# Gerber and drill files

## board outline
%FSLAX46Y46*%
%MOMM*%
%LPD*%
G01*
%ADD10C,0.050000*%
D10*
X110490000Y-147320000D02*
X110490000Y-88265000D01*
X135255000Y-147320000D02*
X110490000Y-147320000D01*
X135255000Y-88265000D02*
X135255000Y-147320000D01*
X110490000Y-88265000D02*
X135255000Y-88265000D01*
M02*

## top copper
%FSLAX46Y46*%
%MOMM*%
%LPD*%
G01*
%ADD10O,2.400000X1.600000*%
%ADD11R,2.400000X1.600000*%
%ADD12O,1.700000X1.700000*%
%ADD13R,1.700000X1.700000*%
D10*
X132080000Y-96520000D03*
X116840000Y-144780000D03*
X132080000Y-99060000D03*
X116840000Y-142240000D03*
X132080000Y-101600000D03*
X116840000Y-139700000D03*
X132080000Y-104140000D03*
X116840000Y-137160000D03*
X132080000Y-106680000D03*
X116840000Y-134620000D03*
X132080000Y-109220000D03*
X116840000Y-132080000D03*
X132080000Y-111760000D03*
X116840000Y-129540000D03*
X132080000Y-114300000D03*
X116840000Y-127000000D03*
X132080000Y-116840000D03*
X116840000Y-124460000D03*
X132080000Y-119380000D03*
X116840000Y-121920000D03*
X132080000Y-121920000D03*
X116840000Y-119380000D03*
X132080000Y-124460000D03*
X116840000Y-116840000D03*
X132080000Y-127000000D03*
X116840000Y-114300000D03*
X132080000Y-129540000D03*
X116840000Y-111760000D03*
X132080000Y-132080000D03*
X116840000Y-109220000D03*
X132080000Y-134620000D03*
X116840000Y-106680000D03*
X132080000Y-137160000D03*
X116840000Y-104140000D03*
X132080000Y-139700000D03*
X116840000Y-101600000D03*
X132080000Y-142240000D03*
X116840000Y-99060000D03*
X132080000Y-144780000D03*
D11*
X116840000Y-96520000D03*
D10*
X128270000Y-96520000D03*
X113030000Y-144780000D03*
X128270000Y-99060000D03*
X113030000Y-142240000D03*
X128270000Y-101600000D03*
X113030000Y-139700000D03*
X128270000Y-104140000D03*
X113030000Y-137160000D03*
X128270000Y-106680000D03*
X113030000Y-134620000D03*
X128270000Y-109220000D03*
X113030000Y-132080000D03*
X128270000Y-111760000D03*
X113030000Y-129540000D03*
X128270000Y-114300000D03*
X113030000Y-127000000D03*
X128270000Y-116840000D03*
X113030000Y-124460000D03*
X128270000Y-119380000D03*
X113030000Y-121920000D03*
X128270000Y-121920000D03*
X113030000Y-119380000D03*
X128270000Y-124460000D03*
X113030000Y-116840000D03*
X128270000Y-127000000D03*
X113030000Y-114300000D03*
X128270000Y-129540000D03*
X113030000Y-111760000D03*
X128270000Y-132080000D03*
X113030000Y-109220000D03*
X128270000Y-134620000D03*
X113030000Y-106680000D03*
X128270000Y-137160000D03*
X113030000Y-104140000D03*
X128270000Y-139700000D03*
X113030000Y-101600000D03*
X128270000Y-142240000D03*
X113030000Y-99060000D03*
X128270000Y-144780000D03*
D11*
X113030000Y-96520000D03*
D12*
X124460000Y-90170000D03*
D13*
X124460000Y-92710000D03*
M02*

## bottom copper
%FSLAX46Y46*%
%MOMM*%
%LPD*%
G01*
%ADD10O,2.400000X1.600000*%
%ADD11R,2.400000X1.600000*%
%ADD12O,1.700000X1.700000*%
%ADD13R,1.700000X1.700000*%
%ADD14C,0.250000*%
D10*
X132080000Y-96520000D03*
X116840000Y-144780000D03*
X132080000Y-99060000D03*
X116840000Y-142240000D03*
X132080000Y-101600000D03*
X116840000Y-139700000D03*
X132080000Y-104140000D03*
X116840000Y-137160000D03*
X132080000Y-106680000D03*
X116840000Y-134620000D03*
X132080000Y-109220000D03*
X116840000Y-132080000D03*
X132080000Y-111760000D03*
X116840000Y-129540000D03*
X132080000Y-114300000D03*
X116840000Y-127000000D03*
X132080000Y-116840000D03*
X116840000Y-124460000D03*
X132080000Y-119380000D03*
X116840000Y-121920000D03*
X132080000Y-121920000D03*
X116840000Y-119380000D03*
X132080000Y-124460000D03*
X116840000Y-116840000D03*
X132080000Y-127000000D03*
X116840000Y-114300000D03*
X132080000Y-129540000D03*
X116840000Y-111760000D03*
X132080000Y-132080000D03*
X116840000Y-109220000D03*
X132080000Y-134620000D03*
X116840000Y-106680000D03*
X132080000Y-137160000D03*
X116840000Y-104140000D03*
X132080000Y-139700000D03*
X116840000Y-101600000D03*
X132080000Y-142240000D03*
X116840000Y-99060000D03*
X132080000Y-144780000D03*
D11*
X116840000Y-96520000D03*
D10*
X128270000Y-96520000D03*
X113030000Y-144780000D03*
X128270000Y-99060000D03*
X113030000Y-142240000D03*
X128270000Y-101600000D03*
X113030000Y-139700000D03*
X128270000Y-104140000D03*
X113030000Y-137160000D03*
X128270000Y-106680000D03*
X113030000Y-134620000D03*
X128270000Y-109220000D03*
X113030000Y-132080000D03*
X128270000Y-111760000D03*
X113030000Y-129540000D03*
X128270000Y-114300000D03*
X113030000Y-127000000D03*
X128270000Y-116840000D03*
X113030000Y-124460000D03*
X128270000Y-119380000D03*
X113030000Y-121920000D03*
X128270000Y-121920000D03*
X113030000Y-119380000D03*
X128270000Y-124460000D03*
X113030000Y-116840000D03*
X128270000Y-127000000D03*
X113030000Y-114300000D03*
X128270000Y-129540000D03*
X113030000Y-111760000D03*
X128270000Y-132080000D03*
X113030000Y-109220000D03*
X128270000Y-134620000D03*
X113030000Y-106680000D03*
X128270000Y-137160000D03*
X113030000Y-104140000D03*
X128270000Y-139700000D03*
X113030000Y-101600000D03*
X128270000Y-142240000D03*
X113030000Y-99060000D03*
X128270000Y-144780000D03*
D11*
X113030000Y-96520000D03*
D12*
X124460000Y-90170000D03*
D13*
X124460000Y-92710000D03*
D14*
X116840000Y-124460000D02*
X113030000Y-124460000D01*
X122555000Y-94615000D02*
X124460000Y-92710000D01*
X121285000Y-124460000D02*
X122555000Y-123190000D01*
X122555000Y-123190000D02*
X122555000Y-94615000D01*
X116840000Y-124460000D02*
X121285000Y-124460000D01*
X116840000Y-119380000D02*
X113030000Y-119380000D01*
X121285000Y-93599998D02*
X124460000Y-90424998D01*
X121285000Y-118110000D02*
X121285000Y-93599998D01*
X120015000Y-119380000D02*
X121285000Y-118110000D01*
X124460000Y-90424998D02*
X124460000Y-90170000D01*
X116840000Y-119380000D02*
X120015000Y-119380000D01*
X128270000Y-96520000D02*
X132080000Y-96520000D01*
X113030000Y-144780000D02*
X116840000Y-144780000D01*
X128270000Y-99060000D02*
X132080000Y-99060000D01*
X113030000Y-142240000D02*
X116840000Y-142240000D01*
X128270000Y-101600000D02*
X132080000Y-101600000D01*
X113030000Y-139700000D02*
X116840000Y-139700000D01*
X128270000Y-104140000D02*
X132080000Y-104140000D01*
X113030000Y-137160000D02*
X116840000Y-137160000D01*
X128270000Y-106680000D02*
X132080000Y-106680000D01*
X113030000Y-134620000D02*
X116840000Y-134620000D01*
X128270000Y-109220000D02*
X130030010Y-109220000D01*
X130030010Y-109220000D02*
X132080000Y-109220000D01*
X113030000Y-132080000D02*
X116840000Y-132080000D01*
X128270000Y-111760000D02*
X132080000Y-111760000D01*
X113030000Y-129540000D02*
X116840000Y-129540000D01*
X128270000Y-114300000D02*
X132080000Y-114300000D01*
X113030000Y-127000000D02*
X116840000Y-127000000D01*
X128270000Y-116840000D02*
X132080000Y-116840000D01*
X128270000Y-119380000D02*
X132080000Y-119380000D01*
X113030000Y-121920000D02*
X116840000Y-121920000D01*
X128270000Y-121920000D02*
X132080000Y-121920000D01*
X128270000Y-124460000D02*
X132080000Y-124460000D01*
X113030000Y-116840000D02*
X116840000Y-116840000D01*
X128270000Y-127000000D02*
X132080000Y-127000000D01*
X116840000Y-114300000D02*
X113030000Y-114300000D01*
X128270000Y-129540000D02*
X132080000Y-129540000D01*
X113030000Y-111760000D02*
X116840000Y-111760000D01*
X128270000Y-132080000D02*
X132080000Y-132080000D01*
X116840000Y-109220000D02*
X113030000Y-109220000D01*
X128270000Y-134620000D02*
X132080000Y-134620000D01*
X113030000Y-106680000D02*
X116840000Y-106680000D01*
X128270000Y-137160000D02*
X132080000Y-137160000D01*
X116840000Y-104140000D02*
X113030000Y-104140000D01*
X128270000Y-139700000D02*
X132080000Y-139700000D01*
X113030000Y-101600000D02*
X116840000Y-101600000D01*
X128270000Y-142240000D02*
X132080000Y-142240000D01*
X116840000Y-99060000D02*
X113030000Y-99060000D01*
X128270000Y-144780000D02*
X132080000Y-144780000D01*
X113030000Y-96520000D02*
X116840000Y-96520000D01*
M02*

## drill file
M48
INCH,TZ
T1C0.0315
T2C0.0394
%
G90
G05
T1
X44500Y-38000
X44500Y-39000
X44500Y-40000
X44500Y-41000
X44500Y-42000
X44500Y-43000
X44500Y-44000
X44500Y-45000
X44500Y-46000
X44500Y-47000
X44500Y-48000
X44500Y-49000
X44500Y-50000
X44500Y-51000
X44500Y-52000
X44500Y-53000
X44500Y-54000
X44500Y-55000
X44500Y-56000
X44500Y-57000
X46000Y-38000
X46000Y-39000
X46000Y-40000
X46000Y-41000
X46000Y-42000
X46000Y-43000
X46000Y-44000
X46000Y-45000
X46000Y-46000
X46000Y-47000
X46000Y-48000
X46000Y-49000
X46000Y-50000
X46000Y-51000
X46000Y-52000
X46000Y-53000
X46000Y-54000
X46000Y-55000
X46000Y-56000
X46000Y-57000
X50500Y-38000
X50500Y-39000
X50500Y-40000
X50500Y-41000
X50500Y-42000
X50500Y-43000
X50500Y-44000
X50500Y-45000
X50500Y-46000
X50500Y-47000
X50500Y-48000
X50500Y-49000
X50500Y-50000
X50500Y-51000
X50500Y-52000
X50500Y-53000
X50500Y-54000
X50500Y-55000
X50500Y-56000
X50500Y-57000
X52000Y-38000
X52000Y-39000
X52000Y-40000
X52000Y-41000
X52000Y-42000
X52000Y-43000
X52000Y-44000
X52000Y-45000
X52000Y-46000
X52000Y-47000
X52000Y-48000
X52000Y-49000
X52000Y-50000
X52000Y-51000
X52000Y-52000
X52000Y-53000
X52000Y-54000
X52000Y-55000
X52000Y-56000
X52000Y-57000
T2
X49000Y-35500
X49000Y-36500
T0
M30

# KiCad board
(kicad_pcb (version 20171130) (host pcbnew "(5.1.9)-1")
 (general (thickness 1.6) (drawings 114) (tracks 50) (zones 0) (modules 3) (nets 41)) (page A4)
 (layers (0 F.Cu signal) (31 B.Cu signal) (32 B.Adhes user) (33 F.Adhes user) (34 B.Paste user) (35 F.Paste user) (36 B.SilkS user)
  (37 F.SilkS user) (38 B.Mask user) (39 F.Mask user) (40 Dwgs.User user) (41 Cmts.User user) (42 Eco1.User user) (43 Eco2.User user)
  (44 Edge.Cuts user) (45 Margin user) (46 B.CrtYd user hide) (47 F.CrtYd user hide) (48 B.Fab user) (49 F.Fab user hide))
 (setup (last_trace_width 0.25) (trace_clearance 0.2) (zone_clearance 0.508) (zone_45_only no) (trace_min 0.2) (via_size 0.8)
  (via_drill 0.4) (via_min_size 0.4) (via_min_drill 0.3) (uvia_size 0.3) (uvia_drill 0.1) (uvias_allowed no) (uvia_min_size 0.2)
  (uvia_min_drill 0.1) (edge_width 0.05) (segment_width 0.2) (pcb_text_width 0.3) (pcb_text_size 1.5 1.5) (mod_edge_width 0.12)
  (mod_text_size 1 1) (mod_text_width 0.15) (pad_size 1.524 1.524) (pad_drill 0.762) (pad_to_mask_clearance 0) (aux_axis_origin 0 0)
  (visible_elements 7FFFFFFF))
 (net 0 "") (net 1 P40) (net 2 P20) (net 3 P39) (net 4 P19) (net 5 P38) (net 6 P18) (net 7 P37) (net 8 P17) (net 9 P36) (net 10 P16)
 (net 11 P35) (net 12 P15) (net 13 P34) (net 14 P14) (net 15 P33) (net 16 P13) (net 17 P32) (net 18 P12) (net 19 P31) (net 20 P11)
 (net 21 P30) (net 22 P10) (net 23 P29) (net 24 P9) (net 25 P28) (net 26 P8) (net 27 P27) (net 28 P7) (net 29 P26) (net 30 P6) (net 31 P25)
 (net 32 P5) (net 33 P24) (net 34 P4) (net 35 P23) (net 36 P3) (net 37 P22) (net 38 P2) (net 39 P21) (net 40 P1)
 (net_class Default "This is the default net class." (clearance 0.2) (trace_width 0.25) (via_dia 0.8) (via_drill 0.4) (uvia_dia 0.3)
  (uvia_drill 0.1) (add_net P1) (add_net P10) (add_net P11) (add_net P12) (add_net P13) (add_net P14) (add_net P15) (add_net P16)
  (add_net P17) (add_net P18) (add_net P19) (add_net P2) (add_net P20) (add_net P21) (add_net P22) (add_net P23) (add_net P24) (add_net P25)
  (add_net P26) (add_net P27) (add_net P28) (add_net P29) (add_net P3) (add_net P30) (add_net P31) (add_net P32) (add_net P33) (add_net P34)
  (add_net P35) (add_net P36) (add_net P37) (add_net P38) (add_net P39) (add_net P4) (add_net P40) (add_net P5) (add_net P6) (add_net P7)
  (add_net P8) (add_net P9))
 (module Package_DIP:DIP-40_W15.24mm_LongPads (layer F.Cu) (at 116.84 96.52)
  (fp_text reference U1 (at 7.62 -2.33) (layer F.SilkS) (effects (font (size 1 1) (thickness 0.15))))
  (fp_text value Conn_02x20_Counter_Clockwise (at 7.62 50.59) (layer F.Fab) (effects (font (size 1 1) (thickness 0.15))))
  (pad 40 thru_hole oval (at 15.24 0) (size 2.4 1.6) (drill 0.8) (layers *.Cu *.Mask) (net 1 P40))
  (pad 20 thru_hole oval (at 0 48.26) (size 2.4 1.6) (drill 0.8) (layers *.Cu *.Mask) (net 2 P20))
  (pad 39 thru_hole oval (at 15.24 2.54) (size 2.4 1.6) (drill 0.8) (layers *.Cu *.Mask) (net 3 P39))
  (pad 19 thru_hole oval (at 0 45.72) (size 2.4 1.6) (drill 0.8) (layers *.Cu *.Mask) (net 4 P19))
  (pad 38 thru_hole oval (at 15.24 5.08) (size 2.4 1.6) (drill 0.8) (layers *.Cu *.Mask) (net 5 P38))
  (pad 18 thru_hole oval (at 0 43.18) (size 2.4 1.6) (drill 0.8) (layers *.Cu *.Mask) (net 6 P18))
  (pad 37 thru_hole oval (at 15.24 7.62) (size 2.4 1.6) (drill 0.8) (layers *.Cu *.Mask) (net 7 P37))
  (pad 17 thru_hole oval (at 0 40.64) (size 2.4 1.6) (drill 0.8) (layers *.Cu *.Mask) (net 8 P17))
  (pad 36 thru_hole oval (at 15.24 10.16) (size 2.4 1.6) (drill 0.8) (layers *.Cu *.Mask) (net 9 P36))
  (pad 16 thru_hole oval (at 0 38.1) (size 2.4 1.6) (drill 0.8) (layers *.Cu *.Mask) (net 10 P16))
  (pad 35 thru_hole oval (at 15.24 12.7) (size 2.4 1.6) (drill 0.8) (layers *.Cu *.Mask) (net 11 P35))
  (pad 15 thru_hole oval (at 0 35.56) (size 2.4 1.6) (drill 0.8) (layers *.Cu *.Mask) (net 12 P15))
  (pad 34 thru_hole oval (at 15.24 15.24) (size 2.4 1.6) (drill 0.8) (layers *.Cu *.Mask) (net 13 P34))
  (pad 14 thru_hole oval (at 0 33.02) (size 2.4 1.6) (drill 0.8) (layers *.Cu *.Mask) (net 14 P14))
  (pad 33 thru_hole oval (at 15.24 17.78) (size 2.4 1.6) (drill 0.8) (layers *.Cu *.Mask) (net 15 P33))
  (pad 13 thru_hole oval (at 0 30.48) (size 2.4 1.6) (drill 0.8) (layers *.Cu *.Mask) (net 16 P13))
  (pad 32 thru_hole oval (at 15.24 20.32) (size 2.4 1.6) (drill 0.8) (layers *.Cu *.Mask) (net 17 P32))
  (pad 12 thru_hole oval (at 0 27.94) (size 2.4 1.6) (drill 0.8) (layers *.Cu *.Mask) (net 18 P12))
  (pad 31 thru_hole oval (at 15.24 22.86) (size 2.4 1.6) (drill 0.8) (layers *.Cu *.Mask) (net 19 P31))
  (pad 11 thru_hole oval (at 0 25.4) (size 2.4 1.6) (drill 0.8) (layers *.Cu *.Mask) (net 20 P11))
  (pad 30 thru_hole oval (at 15.24 25.4) (size 2.4 1.6) (drill 0.8) (layers *.Cu *.Mask) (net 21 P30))
  (pad 10 thru_hole oval (at 0 22.86) (size 2.4 1.6) (drill 0.8) (layers *.Cu *.Mask) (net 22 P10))
  (pad 29 thru_hole oval (at 15.24 27.94) (size 2.4 1.6) (drill 0.8) (layers *.Cu *.Mask) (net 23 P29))
  (pad 9 thru_hole oval (at 0 20.32) (size 2.4 1.6) (drill 0.8) (layers *.Cu *.Mask) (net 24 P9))
  (pad 28 thru_hole oval (at 15.24 30.48) (size 2.4 1.6) (drill 0.8) (layers *.Cu *.Mask) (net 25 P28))
  (pad 8 thru_hole oval (at 0 17.78) (size 2.4 1.6) (drill 0.8) (layers *.Cu *.Mask) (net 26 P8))
  (pad 27 thru_hole oval (at 15.24 33.02) (size 2.4 1.6) (drill 0.8) (layers *.Cu *.Mask) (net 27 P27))
  (pad 7 thru_hole oval (at 0 15.24) (size 2.4 1.6) (drill 0.8) (layers *.Cu *.Mask) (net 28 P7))
  (pad 26 thru_hole oval (at 15.24 35.56) (size 2.4 1.6) (drill 0.8) (layers *.Cu *.Mask) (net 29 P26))
  (pad 6 thru_hole oval (at 0 12.7) (size 2.4 1.6) (drill 0.8) (layers *.Cu *.Mask) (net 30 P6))
  (pad 25 thru_hole oval (at 15.24 38.1) (size 2.4 1.6) (drill 0.8) (layers *.Cu *.Mask) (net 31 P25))
  (pad 5 thru_hole oval (at 0 10.16) (size 2.4 1.6) (drill 0.8) (layers *.Cu *.Mask) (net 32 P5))
  (pad 24 thru_hole oval (at 15.24 40.64) (size 2.4 1.6) (drill 0.8) (layers *.Cu *.Mask) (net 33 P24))
  (pad 4 thru_hole oval (at 0 7.62) (size 2.4 1.6) (drill 0.8) (layers *.Cu *.Mask) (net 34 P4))
  (pad 23 thru_hole oval (at 15.24 43.18) (size 2.4 1.6) (drill 0.8) (layers *.Cu *.Mask) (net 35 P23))
  (pad 3 thru_hole oval (at 0 5.08) (size 2.4 1.6) (drill 0.8) (layers *.Cu *.Mask) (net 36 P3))
  (pad 22 thru_hole oval (at 15.24 45.72) (size 2.4 1.6) (drill 0.8) (layers *.Cu *.Mask) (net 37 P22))
  (pad 2 thru_hole oval (at 0 2.54) (size 2.4 1.6) (drill 0.8) (layers *.Cu *.Mask) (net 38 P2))
  (pad 21 thru_hole oval (at 15.24 48.26) (size 2.4 1.6) (drill 0.8) (layers *.Cu *.Mask) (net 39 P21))
  (pad 1 thru_hole rect (at 0 0) (size 2.4 1.6) (drill 0.8) (layers *.Cu *.Mask) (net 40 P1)))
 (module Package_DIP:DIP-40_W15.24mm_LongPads (layer F.Cu) (at 113.03 96.52)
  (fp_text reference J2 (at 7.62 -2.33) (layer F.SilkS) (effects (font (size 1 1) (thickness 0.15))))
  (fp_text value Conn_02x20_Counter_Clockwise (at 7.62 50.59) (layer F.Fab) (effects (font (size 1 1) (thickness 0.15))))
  (pad 40 thru_hole oval (at 15.24 0) (size 2.4 1.6) (drill 0.8) (layers *.Cu *.Mask) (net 1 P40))
  (pad 20 thru_hole oval (at 0 48.26) (size 2.4 1.6) (drill 0.8) (layers *.Cu *.Mask) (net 2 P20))
  (pad 39 thru_hole oval (at 15.24 2.54) (size 2.4 1.6) (drill 0.8) (layers *.Cu *.Mask) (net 3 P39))
  (pad 19 thru_hole oval (at 0 45.72) (size 2.4 1.6) (drill 0.8) (layers *.Cu *.Mask) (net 4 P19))
  (pad 38 thru_hole oval (at 15.24 5.08) (size 2.4 1.6) (drill 0.8) (layers *.Cu *.Mask) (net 5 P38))
  (pad 18 thru_hole oval (at 0 43.18) (size 2.4 1.6) (drill 0.8) (layers *.Cu *.Mask) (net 6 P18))
  (pad 37 thru_hole oval (at 15.24 7.62) (size 2.4 1.6) (drill 0.8) (layers *.Cu *.Mask) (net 7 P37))
  (pad 17 thru_hole oval (at 0 40.64) (size 2.4 1.6) (drill 0.8) (layers *.Cu *.Mask) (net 8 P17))
  (pad 36 thru_hole oval (at 15.24 10.16) (size 2.4 1.6) (drill 0.8) (layers *.Cu *.Mask) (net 9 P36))
  (pad 16 thru_hole oval (at 0 38.1) (size 2.4 1.6) (drill 0.8) (layers *.Cu *.Mask) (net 10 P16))
  (pad 35 thru_hole oval (at 15.24 12.7) (size 2.4 1.6) (drill 0.8) (layers *.Cu *.Mask) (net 11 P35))
  (pad 15 thru_hole oval (at 0 35.56) (size 2.4 1.6) (drill 0.8) (layers *.Cu *.Mask) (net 12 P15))
  (pad 34 thru_hole oval (at 15.24 15.24) (size 2.4 1.6) (drill 0.8) (layers *.Cu *.Mask) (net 13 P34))
  (pad 14 thru_hole oval (at 0 33.02) (size 2.4 1.6) (drill 0.8) (layers *.Cu *.Mask) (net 14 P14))
  (pad 33 thru_hole oval (at 15.24 17.78) (size 2.4 1.6) (drill 0.8) (layers *.Cu *.Mask) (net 15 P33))
  (pad 13 thru_hole oval (at 0 30.48) (size 2.4 1.6) (drill 0.8) (layers *.Cu *.Mask) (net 16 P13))
  (pad 32 thru_hole oval (at 15.24 20.32) (size 2.4 1.6) (drill 0.8) (layers *.Cu *.Mask) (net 17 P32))
  (pad 12 thru_hole oval (at 0 27.94) (size 2.4 1.6) (drill 0.8) (layers *.Cu *.Mask) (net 18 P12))
  (pad 31 thru_hole oval (at 15.24 22.86) (size 2.4 1.6) (drill 0.8) (layers *.Cu *.Mask) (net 19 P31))
  (pad 11 thru_hole oval (at 0 25.4) (size 2.4 1.6) (drill 0.8) (layers *.Cu *.Mask) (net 20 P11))
  (pad 30 thru_hole oval (at 15.24 25.4) (size 2.4 1.6) (drill 0.8) (layers *.Cu *.Mask) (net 21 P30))
  (pad 10 thru_hole oval (at 0 22.86) (size 2.4 1.6) (drill 0.8) (layers *.Cu *.Mask) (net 22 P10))
  (pad 29 thru_hole oval (at 15.24 27.94) (size 2.4 1.6) (drill 0.8) (layers *.Cu *.Mask) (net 23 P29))
  (pad 9 thru_hole oval (at 0 20.32) (size 2.4 1.6) (drill 0.8) (layers *.Cu *.Mask) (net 24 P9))
  (pad 28 thru_hole oval (at 15.24 30.48) (size 2.4 1.6) (drill 0.8) (layers *.Cu *.Mask) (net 25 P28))
  (pad 8 thru_hole oval (at 0 17.78) (size 2.4 1.6) (drill 0.8) (layers *.Cu *.Mask) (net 26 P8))
  (pad 27 thru_hole oval (at 15.24 33.02) (size 2.4 1.6) (drill 0.8) (layers *.Cu *.Mask) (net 27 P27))
  (pad 7 thru_hole oval (at 0 15.24) (size 2.4 1.6) (drill 0.8) (layers *.Cu *.Mask) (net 28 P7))
  (pad 26 thru_hole oval (at 15.24 35.56) (size 2.4 1.6) (drill 0.8) (layers *.Cu *.Mask) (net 29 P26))
  (pad 6 thru_hole oval (at 0 12.7) (size 2.4 1.6) (drill 0.8) (layers *.Cu *.Mask) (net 30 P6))
  (pad 25 thru_hole oval (at 15.24 38.1) (size 2.4 1.6) (drill 0.8) (layers *.Cu *.Mask) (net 31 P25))
  (pad 5 thru_hole oval (at 0 10.16) (size 2.4 1.6) (drill 0.8) (layers *.Cu *.Mask) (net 32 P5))
  (pad 24 thru_hole oval (at 15.24 40.64) (size 2.4 1.6) (drill 0.8) (layers *.Cu *.Mask) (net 33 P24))
  (pad 4 thru_hole oval (at 0 7.62) (size 2.4 1.6) (drill 0.8) (layers *.Cu *.Mask) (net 34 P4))
  (pad 23 thru_hole oval (at 15.24 43.18) (size 2.4 1.6) (drill 0.8) (layers *.Cu *.Mask) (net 35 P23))
  (pad 3 thru_hole oval (at 0 5.08) (size 2.4 1.6) (drill 0.8) (layers *.Cu *.Mask) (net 36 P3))
  (pad 22 thru_hole oval (at 15.24 45.72) (size 2.4 1.6) (drill 0.8) (layers *.Cu *.Mask) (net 37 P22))
  (pad 2 thru_hole oval (at 0 2.54) (size 2.4 1.6) (drill 0.8) (layers *.Cu *.Mask) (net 38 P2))
  (pad 21 thru_hole oval (at 15.24 48.26) (size 2.4 1.6) (drill 0.8) (layers *.Cu *.Mask) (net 39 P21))
  (pad 1 thru_hole rect (at 0 0) (size 2.4 1.6) (drill 0.8) (layers *.Cu *.Mask) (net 40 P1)))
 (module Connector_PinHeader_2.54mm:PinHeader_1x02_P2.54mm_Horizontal (layer F.Cu) (at 124.46 92.71 180)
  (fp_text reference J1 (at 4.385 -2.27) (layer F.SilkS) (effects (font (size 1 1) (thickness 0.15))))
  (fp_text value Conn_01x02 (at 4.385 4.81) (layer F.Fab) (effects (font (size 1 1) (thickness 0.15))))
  (pad 2 thru_hole oval (at 0 2.54 180) (size 1.7 1.7) (drill 1) (layers *.Cu *.Mask) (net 22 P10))
  (pad 1 thru_hole rect (at 0 0 180) (size 1.7 1.7) (drill 1) (layers *.Cu *.Mask) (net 18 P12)))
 (gr_line (start 110.49 147.32) (end 110.49 88.265) (layer Edge.Cuts) (width 0.05))
 (gr_line (start 135.255 147.32) (end 110.49 147.32) (layer Edge.Cuts) (width 0.05))
 (gr_line (start 135.255 88.265) (end 135.255 147.32) (layer Edge.Cuts) (width 0.05))
 (gr_line (start 110.49 88.265) (end 135.255 88.265) (layer Edge.Cuts) (width 0.05))
 (segment (start 116.84 124.46) (end 113.03 124.46) (width 0.25) (layer B.Cu) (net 18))
 (segment (start 122.555 94.615) (end 124.46 92.71) (width 0.25) (layer B.Cu) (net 18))
 (segment (start 121.285 124.46) (end 122.555 123.19) (width 0.25) (layer B.Cu) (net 18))
 (segment (start 122.555 123.19) (end 122.555 94.615) (width 0.25) (layer B.Cu) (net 18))
 (segment (start 116.84 124.46) (end 121.285 124.46) (width 0.25) (layer B.Cu) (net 18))
 (segment (start 116.84 119.38) (end 113.03 119.38) (width 0.25) (layer B.Cu) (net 22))
 (segment (start 121.285 93.599998) (end 124.46 90.424998) (width 0.25) (layer B.Cu) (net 22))
 (segment (start 121.285 118.11) (end 121.285 93.599998) (width 0.25) (layer B.Cu) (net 22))
 (segment (start 120.015 119.38) (end 121.285 118.11) (width 0.25) (layer B.Cu) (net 22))
 (segment (start 124.46 90.424998) (end 124.46 90.17) (width 0.25) (layer B.Cu) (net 22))
 (segment (start 116.84 119.38) (end 120.015 119.38) (width 0.25) (layer B.Cu) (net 22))
 (segment (start 128.27 96.52) (end 132.08 96.52) (width 0.25) (layer B.Cu) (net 1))
 (segment (start 113.03 144.78) (end 116.84 144.78) (width 0.25) (layer B.Cu) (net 2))
 (segment (start 128.27 99.06) (end 132.08 99.06) (width 0.25) (layer B.Cu) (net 3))
 (segment (start 113.03 142.24) (end 116.84 142.24) (width 0.25) (layer B.Cu) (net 4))
 (segment (start 128.27 101.6) (end 132.08 101.6) (width 0.25) (layer B.Cu) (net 5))
 (segment (start 113.03 139.7) (end 116.84 139.7) (width 0.25) (layer B.Cu) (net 6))
 (segment (start 128.27 104.14) (end 132.08 104.14) (width 0.25) (layer B.Cu) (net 7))
 (segment (start 113.03 137.16) (end 116.84 137.16) (width 0.25) (layer B.Cu) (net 8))
 (segment (start 128.27 106.68) (end 132.08 106.68) (width 0.25) (layer B.Cu) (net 9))
 (segment (start 113.03 134.62) (end 116.84 134.62) (width 0.25) (layer B.Cu) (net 10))
 (segment (start 128.27 109.22) (end 130.03001 109.22) (width 0.25) (layer B.Cu) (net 11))
 (segment (start 130.03001 109.22) (end 132.08 109.22) (width 0.25) (layer B.Cu) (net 11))
 (segment (start 113.03 132.08) (end 116.84 132.08) (width 0.25) (layer B.Cu) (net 12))
 (segment (start 128.27 111.76) (end 132.08 111.76) (width 0.25) (layer B.Cu) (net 13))
 (segment (start 113.03 129.54) (end 116.84 129.54) (width 0.25) (layer B.Cu) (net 14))
 (segment (start 128.27 114.3) (end 132.08 114.3) (width 0.25) (layer B.Cu) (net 15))
 (segment (start 113.03 127) (end 116.84 127) (width 0.25) (layer B.Cu) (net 16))
 (segment (start 128.27 116.84) (end 132.08 116.84) (width 0.25) (layer B.Cu) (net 17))
 (segment (start 128.27 119.38) (end 132.08 119.38) (width 0.25) (layer B.Cu) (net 19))
 (segment (start 113.03 121.92) (end 116.84 121.92) (width 0.25) (layer B.Cu) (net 20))
 (segment (start 128.27 121.92) (end 132.08 121.92) (width 0.25) (layer B.Cu) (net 21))
 (segment (start 128.27 124.46) (end 132.08 124.46) (width 0.25) (layer B.Cu) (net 23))
 (segment (start 113.03 116.84) (end 116.84 116.84) (width 0.25) (layer B.Cu) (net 24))
 (segment (start 128.27 127) (end 132.08 127) (width 0.25) (layer B.Cu) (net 25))
 (segment (start 116.84 114.3) (end 113.03 114.3) (width 0.25) (layer B.Cu) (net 26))
 (segment (start 128.27 129.54) (end 132.08 129.54) (width 0.25) (layer B.Cu) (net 27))
 (segment (start 113.03 111.76) (end 116.84 111.76) (width 0.25) (layer B.Cu) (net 28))
 (segment (start 128.27 132.08) (end 132.08 132.08) (width 0.25) (layer B.Cu) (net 29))
 (segment (start 116.84 109.22) (end 113.03 109.22) (width 0.25) (layer B.Cu) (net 30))
 (segment (start 128.27 134.62) (end 132.08 134.62) (width 0.25) (layer B.Cu) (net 31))
 (segment (start 113.03 106.68) (end 116.84 106.68) (width 0.25) (layer B.Cu) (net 32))
 (segment (start 128.27 137.16) (end 132.08 137.16) (width 0.25) (layer B.Cu) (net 33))
 (segment (start 116.84 104.14) (end 113.03 104.14) (width 0.25) (layer B.Cu) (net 34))
 (segment (start 128.27 139.7) (end 132.08 139.7) (width 0.25) (layer B.Cu) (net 35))
 (segment (start 113.03 101.6) (end 116.84 101.6) (width 0.25) (layer B.Cu) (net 36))
 (segment (start 128.27 142.24) (end 132.08 142.24) (width 0.25) (layer B.Cu) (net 37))
 (segment (start 116.84 99.06) (end 113.03 99.06) (width 0.25) (layer B.Cu) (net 38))
 (segment (start 128.27 144.78) (end 132.08 144.78) (width 0.25) (layer B.Cu) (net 39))
 (segment (start 113.03 96.52) (end 116.84 96.52) (width 0.25) (layer B.Cu) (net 40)))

